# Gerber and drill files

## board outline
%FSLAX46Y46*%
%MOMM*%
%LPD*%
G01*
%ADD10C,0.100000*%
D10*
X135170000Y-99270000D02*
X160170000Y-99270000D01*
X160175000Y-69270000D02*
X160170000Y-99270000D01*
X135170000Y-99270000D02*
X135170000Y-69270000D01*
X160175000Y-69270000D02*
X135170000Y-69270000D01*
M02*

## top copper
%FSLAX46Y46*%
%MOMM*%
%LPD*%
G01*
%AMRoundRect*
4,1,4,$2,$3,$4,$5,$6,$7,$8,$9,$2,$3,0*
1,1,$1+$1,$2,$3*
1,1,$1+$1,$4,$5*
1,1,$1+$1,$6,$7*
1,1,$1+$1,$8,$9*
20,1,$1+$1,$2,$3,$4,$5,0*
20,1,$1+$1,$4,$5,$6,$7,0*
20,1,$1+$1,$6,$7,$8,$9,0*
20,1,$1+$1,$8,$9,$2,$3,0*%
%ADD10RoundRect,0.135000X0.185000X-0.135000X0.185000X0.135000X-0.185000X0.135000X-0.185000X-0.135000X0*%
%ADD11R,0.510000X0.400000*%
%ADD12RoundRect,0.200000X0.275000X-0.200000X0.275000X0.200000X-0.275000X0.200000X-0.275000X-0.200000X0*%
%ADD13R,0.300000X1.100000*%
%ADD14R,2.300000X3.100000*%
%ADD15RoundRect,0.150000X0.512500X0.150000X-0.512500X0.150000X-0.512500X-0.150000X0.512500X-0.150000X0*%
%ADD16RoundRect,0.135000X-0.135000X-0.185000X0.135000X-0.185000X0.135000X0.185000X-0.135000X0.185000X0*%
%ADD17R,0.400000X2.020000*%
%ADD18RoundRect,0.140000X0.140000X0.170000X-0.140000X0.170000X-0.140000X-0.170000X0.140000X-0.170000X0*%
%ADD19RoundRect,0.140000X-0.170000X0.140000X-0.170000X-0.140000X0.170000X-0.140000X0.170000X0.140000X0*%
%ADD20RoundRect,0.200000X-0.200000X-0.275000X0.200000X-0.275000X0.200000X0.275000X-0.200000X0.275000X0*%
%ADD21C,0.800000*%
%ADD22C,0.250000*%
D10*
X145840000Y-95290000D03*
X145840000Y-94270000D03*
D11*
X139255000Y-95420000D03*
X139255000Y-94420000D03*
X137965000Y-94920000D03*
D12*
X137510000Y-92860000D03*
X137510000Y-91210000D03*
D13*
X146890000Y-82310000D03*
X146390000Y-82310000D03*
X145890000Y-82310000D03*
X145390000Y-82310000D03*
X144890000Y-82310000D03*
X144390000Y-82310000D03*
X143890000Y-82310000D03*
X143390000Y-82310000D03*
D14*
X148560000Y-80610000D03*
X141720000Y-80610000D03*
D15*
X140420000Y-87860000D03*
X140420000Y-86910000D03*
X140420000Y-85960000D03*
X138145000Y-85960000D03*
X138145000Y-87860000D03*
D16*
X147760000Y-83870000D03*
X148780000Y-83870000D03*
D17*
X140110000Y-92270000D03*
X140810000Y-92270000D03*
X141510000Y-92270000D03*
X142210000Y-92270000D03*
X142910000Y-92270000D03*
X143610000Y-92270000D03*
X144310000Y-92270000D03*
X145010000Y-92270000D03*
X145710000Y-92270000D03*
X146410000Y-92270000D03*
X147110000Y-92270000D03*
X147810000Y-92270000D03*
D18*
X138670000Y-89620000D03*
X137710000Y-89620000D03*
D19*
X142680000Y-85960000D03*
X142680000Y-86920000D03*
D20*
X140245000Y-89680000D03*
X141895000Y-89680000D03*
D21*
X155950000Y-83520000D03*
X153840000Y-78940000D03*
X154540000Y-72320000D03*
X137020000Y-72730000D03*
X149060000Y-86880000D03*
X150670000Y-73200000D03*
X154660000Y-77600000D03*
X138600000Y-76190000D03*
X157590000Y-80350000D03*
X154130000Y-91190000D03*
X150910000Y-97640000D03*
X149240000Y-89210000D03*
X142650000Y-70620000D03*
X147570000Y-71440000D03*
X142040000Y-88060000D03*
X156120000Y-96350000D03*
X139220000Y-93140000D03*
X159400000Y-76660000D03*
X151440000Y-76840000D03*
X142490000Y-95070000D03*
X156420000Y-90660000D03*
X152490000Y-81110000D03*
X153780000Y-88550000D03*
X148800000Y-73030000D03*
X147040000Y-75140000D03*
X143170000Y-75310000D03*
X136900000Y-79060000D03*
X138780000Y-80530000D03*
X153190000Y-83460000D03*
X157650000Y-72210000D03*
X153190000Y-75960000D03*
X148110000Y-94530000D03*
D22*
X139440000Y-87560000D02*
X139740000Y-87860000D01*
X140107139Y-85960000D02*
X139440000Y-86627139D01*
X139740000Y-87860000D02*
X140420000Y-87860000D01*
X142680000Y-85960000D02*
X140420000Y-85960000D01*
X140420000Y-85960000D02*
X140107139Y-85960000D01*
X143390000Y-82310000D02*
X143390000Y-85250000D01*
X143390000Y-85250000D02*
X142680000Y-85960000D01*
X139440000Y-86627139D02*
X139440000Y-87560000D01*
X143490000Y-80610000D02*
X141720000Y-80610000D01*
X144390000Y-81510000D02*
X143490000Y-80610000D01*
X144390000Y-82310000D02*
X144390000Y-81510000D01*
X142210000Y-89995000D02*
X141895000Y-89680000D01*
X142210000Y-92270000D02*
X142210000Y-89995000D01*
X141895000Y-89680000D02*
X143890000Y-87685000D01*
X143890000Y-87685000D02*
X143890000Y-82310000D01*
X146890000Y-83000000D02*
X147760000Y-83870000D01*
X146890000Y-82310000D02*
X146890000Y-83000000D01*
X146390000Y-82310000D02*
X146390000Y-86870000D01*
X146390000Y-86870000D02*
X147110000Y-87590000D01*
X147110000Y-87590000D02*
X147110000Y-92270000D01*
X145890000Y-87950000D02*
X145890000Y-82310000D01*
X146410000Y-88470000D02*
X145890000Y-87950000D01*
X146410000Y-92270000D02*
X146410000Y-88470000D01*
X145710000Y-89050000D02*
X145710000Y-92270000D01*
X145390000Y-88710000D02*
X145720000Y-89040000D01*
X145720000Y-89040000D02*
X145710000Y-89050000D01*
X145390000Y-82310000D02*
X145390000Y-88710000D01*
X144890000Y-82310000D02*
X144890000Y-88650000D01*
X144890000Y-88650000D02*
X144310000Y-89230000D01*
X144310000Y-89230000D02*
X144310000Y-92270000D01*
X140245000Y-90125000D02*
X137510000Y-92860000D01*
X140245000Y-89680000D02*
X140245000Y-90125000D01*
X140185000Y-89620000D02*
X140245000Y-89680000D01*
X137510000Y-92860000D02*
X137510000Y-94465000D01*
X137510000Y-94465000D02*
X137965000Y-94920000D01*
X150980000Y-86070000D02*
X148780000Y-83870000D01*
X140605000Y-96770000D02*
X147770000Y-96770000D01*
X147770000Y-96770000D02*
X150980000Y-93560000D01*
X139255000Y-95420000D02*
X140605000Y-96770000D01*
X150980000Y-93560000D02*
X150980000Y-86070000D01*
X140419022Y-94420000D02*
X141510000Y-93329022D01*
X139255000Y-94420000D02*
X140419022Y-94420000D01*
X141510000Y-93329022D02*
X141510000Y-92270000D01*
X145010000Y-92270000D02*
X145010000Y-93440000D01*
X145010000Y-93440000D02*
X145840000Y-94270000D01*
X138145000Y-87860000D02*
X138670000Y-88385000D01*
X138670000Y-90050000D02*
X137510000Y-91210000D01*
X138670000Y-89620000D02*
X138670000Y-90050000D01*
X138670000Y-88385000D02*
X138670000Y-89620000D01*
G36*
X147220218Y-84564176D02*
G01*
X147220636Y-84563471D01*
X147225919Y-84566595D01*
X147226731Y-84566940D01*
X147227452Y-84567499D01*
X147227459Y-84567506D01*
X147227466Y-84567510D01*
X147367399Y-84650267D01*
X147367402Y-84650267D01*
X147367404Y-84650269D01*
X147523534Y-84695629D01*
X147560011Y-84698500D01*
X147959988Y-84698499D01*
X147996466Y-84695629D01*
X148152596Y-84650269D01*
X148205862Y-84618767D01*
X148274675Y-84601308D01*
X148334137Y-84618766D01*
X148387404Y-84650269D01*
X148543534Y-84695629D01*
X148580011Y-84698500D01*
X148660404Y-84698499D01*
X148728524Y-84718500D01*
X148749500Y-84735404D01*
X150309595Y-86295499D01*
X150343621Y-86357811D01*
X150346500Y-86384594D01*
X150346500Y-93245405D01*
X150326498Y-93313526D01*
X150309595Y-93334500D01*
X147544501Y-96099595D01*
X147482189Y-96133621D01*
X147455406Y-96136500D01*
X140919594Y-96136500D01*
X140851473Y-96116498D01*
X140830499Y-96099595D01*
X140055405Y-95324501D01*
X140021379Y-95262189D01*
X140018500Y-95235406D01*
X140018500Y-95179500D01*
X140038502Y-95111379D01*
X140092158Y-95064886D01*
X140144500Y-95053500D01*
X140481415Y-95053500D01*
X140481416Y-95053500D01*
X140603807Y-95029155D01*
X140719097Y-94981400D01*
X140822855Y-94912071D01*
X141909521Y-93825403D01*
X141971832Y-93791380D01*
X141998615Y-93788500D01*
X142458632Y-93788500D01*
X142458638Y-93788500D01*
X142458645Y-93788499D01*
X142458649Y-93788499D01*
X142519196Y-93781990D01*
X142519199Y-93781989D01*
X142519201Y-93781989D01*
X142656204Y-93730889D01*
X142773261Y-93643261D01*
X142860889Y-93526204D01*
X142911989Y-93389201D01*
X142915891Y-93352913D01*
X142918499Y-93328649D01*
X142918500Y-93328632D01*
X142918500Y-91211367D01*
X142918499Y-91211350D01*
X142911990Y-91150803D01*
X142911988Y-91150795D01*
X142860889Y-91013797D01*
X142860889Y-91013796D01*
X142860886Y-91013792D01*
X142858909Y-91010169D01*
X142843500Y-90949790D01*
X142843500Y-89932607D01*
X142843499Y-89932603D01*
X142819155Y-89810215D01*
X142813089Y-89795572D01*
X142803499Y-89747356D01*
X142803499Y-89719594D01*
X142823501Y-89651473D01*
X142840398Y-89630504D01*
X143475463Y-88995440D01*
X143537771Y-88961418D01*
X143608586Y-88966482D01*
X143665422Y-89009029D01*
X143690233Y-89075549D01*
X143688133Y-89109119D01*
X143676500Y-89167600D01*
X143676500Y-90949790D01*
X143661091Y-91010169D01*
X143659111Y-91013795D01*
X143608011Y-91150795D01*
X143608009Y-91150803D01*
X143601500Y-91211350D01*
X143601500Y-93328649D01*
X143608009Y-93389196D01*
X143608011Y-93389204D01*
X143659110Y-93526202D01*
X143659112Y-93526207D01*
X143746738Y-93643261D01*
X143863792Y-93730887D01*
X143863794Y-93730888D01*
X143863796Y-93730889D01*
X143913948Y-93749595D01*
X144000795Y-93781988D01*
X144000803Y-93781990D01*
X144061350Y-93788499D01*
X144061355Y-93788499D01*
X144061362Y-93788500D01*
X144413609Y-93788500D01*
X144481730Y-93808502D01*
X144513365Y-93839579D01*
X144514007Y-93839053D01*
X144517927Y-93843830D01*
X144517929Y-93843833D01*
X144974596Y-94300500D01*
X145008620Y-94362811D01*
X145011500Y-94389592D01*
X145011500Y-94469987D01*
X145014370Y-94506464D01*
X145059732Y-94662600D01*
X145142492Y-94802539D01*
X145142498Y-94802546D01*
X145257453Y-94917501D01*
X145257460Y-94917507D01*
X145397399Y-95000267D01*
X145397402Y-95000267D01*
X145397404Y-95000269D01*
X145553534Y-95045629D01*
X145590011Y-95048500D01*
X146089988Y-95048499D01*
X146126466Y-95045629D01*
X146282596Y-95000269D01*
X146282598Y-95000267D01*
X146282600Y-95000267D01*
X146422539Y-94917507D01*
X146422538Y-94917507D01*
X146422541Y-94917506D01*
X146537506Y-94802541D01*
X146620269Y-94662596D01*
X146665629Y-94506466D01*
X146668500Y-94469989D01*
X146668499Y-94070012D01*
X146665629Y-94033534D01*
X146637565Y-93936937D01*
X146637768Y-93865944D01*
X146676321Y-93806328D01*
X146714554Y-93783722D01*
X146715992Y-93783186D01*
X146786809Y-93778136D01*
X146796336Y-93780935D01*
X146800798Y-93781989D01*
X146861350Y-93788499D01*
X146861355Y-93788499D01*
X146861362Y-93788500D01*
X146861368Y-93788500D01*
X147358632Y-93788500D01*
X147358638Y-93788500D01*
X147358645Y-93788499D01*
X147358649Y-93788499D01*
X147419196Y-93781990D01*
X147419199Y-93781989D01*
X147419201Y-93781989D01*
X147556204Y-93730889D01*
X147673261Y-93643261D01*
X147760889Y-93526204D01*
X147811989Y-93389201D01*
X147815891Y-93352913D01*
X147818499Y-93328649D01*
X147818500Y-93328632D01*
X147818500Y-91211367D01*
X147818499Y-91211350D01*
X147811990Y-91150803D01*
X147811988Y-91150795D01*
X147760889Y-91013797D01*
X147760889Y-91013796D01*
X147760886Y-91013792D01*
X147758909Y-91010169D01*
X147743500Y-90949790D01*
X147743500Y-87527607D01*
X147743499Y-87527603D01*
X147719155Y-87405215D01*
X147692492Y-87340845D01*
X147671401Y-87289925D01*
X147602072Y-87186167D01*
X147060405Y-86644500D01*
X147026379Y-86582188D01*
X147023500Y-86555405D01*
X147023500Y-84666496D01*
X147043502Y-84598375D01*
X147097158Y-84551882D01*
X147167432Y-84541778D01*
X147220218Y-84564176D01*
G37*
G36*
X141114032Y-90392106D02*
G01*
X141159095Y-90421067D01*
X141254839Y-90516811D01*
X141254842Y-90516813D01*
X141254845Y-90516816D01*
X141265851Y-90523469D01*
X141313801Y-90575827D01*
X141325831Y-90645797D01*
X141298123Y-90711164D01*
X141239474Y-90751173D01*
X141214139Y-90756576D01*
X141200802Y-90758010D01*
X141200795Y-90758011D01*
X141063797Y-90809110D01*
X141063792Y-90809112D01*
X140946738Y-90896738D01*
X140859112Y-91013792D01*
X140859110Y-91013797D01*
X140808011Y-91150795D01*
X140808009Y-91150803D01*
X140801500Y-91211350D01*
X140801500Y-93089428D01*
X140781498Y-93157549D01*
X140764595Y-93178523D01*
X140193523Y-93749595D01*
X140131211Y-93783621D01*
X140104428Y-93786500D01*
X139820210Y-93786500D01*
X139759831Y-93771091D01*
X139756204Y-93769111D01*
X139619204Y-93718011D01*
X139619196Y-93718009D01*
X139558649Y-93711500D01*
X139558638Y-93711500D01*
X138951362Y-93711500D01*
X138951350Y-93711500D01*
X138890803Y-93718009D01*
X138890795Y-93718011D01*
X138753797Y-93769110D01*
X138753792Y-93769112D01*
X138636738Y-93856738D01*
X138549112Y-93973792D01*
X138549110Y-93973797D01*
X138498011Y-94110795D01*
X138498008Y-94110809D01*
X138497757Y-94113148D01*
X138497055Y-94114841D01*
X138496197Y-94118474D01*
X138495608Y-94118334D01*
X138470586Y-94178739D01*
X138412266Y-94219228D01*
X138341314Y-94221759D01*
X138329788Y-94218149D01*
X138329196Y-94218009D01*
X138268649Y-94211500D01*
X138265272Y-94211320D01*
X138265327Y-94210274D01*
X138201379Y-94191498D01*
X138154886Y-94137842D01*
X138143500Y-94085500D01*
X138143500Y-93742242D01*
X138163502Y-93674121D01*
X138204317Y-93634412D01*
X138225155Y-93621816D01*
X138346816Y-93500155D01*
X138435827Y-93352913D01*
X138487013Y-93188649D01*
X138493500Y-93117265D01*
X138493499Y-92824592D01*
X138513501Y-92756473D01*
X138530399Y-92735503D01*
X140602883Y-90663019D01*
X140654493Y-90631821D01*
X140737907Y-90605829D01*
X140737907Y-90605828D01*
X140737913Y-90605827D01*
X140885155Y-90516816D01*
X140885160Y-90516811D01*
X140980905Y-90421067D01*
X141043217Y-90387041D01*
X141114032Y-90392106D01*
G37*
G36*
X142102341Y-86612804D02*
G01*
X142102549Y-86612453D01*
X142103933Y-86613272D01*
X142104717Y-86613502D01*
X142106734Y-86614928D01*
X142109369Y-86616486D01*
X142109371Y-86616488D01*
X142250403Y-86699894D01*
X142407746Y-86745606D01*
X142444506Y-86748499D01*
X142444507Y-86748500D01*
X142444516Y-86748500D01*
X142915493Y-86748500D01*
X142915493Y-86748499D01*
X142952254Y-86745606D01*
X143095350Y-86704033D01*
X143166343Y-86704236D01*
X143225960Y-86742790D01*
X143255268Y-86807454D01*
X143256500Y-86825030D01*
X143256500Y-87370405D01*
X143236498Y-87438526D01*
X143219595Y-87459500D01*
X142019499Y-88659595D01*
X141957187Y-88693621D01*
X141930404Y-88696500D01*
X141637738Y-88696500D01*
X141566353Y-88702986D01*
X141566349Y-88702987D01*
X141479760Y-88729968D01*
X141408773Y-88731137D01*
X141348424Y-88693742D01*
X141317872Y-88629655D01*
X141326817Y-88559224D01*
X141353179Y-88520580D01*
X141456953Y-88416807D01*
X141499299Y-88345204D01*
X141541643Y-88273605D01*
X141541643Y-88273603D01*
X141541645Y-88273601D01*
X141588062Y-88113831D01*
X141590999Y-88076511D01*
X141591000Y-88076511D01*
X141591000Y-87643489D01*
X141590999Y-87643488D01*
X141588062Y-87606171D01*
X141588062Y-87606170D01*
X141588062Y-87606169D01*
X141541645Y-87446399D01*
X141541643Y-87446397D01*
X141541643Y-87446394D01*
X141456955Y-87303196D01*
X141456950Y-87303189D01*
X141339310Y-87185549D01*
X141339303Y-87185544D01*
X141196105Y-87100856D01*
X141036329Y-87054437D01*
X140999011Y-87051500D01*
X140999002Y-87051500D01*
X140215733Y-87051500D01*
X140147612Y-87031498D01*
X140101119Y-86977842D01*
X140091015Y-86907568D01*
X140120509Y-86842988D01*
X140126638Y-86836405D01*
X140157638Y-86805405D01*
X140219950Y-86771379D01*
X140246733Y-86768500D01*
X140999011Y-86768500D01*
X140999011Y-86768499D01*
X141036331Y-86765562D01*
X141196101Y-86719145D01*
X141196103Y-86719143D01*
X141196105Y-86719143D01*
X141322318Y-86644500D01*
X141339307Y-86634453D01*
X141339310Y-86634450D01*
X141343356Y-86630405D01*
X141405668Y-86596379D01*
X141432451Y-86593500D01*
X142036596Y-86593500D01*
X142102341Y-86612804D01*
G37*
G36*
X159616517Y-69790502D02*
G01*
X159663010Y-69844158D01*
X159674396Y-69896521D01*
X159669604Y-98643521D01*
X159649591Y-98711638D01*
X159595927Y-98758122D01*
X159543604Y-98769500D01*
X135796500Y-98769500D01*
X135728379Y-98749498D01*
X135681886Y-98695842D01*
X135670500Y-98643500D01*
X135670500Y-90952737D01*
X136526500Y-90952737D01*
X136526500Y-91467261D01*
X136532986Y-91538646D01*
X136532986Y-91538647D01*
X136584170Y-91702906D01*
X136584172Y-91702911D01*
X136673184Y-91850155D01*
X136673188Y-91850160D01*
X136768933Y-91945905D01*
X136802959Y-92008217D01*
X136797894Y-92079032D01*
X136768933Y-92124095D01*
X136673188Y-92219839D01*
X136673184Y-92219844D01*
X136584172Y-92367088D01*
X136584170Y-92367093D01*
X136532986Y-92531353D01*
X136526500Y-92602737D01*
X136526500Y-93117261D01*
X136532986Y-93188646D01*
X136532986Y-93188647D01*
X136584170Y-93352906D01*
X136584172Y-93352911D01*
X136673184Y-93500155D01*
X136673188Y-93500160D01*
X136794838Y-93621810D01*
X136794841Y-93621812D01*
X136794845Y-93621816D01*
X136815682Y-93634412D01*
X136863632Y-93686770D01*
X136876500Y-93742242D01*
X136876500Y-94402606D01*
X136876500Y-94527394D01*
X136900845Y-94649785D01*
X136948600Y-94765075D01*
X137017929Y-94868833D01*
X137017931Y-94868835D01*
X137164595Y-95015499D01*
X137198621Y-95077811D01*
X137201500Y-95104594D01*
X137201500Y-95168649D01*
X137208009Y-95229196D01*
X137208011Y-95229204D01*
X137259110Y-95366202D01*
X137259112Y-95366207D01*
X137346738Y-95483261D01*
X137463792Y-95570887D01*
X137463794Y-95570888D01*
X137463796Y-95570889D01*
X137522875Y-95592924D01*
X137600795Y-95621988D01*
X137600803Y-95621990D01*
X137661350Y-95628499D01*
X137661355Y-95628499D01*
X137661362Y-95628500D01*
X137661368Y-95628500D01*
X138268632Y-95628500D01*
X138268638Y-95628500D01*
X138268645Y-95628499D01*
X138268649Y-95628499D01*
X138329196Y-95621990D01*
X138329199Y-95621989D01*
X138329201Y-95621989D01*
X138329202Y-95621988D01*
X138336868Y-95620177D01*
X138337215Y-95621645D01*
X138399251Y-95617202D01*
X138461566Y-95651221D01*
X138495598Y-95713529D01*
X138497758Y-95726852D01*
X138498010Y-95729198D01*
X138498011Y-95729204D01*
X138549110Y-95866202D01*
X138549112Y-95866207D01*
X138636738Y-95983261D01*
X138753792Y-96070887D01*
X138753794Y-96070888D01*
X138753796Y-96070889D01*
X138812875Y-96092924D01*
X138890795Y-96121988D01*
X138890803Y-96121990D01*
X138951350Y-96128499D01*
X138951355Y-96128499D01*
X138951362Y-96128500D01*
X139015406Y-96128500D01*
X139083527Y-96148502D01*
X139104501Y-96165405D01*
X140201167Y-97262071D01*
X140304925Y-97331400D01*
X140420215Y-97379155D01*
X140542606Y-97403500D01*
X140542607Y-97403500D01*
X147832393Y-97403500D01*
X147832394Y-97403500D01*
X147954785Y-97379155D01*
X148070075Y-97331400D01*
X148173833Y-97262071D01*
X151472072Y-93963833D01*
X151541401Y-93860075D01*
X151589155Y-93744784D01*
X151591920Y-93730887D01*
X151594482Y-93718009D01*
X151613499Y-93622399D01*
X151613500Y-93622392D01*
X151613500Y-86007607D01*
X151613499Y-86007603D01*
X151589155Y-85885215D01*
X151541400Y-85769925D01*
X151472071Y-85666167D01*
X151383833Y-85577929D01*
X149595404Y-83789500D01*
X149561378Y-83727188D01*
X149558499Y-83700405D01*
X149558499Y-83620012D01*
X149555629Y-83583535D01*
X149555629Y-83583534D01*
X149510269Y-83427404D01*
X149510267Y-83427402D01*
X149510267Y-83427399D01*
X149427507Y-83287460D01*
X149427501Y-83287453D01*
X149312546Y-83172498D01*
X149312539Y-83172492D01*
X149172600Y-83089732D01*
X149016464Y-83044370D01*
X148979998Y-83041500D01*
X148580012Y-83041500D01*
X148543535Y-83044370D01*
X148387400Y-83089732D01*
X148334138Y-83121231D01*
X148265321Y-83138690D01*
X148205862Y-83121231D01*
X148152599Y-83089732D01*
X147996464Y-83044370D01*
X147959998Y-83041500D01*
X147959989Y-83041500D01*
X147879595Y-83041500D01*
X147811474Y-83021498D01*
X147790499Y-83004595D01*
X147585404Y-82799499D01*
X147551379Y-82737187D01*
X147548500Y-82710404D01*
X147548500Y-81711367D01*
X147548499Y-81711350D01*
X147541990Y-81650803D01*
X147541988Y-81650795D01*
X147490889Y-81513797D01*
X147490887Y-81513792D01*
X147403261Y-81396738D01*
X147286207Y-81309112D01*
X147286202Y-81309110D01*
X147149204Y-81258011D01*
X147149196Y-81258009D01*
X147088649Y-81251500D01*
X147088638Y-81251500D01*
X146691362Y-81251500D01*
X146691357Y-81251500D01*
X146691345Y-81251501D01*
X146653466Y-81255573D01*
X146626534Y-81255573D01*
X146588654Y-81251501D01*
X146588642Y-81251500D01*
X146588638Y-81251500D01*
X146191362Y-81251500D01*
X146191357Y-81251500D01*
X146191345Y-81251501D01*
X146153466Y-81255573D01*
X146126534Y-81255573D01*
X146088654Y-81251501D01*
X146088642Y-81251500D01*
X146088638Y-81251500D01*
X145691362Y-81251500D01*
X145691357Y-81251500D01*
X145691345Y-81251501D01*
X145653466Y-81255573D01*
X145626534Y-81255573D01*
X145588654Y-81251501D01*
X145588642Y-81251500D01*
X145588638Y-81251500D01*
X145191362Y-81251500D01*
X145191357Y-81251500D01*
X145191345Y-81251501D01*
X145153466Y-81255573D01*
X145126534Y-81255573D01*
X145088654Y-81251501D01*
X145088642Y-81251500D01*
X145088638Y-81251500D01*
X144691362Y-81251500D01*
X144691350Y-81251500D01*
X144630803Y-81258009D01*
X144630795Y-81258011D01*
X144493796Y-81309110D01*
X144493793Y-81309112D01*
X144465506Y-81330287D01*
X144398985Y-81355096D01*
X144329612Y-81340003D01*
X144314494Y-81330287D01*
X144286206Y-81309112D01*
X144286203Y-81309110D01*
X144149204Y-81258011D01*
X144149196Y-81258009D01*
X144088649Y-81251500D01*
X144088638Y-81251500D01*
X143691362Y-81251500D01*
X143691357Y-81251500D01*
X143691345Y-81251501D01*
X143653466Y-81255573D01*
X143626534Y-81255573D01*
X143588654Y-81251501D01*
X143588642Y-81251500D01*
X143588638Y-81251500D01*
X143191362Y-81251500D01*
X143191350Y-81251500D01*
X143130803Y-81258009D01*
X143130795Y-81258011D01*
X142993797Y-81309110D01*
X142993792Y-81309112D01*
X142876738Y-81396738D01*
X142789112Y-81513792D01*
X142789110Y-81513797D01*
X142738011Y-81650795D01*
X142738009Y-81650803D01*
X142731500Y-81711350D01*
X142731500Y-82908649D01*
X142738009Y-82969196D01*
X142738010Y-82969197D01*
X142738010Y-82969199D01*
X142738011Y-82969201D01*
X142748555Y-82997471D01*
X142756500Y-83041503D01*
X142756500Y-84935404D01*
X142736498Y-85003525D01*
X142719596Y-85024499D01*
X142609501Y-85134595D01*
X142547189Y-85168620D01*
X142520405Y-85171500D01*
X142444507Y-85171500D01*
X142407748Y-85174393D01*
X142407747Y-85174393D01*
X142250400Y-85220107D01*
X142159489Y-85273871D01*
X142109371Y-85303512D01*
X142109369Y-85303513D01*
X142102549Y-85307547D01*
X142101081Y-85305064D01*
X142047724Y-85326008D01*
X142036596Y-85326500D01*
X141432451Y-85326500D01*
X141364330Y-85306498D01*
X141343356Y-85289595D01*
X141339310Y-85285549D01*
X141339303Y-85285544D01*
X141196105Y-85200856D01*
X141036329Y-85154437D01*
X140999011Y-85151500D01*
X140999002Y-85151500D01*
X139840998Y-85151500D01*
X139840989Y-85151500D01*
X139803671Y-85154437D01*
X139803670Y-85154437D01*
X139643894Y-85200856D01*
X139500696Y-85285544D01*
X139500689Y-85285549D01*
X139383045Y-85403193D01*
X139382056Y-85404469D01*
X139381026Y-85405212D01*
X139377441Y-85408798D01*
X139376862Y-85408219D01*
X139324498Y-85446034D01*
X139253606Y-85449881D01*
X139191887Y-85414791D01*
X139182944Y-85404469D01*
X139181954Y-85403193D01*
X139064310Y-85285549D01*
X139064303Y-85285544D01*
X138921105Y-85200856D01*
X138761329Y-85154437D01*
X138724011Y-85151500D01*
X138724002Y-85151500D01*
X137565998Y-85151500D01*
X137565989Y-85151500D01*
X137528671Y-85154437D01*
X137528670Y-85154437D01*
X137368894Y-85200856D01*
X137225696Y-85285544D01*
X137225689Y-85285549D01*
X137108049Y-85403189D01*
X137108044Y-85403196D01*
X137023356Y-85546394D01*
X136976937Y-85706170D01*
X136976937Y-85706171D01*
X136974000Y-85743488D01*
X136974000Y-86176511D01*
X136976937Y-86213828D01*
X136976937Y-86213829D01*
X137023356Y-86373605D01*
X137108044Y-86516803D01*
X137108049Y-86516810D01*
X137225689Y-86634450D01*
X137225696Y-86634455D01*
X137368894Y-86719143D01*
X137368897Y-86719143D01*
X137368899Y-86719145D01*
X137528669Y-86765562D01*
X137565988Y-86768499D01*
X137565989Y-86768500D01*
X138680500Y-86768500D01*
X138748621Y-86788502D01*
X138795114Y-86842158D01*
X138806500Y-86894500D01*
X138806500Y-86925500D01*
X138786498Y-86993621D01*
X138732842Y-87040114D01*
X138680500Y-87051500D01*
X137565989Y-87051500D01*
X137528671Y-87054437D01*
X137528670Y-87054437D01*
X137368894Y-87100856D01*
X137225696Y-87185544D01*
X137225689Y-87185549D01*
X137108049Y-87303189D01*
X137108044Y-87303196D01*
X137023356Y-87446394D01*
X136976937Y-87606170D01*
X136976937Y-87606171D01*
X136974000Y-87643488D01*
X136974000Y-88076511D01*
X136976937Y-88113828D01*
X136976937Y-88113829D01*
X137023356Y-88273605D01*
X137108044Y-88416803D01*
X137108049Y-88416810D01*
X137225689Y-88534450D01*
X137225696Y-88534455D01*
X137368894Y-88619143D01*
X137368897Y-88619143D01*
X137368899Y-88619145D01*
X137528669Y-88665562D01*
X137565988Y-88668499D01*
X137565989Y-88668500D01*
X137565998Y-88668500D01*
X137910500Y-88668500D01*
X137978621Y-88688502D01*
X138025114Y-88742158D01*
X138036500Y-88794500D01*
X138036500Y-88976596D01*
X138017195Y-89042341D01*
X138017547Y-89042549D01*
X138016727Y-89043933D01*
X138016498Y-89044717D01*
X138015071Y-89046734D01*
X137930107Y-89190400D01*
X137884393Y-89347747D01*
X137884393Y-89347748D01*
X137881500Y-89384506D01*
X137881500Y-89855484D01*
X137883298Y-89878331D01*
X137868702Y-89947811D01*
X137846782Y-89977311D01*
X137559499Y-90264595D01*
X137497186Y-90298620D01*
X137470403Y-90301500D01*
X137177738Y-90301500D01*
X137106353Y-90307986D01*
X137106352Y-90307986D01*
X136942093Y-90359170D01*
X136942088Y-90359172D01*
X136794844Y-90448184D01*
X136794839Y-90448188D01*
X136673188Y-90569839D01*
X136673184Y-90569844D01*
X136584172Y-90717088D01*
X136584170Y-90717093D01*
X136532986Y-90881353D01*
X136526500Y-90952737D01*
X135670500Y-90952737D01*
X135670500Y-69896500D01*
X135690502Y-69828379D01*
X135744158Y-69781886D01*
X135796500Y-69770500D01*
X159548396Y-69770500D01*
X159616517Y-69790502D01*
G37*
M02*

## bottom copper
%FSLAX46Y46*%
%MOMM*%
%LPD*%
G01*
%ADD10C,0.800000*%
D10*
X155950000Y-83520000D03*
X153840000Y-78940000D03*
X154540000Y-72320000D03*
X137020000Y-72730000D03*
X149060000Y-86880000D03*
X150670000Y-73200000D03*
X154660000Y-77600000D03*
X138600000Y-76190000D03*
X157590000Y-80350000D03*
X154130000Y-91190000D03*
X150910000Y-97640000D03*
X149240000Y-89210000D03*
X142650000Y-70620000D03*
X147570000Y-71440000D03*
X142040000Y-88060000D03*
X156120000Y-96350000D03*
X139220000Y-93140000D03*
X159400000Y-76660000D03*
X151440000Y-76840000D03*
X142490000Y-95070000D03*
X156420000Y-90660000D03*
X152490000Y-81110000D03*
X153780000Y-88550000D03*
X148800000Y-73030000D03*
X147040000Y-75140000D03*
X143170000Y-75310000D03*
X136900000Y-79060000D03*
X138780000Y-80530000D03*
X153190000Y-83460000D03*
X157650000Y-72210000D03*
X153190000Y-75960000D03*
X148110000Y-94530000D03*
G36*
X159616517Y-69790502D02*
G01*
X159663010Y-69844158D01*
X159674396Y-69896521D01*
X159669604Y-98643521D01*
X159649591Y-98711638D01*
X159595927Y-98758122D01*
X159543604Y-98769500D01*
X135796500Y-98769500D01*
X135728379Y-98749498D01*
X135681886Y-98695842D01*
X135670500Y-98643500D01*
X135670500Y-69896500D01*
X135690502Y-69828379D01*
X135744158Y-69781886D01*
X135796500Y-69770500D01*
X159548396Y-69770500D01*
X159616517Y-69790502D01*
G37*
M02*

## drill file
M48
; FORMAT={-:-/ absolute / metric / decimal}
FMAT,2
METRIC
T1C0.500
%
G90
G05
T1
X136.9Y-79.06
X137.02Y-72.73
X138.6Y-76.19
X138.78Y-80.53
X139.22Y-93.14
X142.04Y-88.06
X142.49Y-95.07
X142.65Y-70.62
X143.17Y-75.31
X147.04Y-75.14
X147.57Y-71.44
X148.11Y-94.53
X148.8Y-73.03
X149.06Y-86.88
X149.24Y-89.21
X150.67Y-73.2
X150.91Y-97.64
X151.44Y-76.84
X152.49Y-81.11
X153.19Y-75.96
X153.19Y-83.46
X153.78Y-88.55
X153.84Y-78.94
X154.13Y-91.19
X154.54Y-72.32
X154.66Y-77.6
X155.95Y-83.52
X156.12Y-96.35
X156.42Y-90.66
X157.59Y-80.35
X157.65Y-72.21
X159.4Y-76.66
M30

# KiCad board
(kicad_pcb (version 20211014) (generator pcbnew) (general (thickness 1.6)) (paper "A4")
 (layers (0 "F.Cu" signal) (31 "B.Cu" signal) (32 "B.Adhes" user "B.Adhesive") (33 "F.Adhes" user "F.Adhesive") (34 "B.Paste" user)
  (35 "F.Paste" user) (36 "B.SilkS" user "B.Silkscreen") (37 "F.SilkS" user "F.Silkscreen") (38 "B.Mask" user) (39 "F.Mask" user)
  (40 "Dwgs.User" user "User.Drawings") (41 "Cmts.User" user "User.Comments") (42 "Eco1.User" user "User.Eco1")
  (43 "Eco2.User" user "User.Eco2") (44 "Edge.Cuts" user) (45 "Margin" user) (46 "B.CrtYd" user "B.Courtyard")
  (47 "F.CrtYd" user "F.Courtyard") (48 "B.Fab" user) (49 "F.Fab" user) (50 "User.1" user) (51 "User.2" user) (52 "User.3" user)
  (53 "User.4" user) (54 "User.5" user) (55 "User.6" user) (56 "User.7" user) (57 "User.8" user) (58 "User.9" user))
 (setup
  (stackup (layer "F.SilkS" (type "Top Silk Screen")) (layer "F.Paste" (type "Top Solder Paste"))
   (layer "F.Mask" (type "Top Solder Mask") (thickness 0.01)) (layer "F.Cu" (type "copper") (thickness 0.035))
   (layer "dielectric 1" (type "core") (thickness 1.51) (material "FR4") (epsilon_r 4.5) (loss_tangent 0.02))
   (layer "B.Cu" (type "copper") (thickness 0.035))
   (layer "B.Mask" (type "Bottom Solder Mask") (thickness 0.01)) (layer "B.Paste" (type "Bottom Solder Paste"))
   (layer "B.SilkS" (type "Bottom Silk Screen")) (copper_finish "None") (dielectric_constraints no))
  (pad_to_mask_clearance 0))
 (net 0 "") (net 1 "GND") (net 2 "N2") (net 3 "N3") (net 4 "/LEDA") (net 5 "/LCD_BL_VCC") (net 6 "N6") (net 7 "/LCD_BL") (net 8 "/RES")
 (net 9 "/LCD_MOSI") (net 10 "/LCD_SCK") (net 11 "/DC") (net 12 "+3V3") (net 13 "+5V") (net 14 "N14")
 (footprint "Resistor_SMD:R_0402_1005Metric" (layer "F.Cu") (at 145.84 94.78 90)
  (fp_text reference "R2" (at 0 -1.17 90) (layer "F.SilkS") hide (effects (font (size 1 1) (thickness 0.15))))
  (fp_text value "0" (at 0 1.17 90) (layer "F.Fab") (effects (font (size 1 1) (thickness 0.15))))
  (pad "1" smd roundrect (at -0.51 0 90) (size 0.54 0.64) (layers "F.Cu" "F.Paste" "F.Mask") (roundrect_rratio 0.25) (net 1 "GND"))
  (pad "2" smd roundrect (at 0.51 0 90) (size 0.54 0.64) (layers "F.Cu" "F.Paste" "F.Mask") (roundrect_rratio 0.25) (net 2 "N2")))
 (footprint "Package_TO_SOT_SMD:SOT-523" (layer "F.Cu") (at 138.61 94.92 180)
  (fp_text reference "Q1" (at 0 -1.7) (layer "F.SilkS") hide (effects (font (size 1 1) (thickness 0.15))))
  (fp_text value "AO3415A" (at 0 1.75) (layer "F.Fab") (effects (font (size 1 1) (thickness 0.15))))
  (pad "1" smd rect (at -0.645 -0.5) (size 0.51 0.4) (layers "F.Cu" "F.Paste" "F.Mask") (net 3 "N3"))
  (pad "2" smd rect (at -0.645 0.5) (size 0.51 0.4) (layers "F.Cu" "F.Paste" "F.Mask") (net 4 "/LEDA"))
  (pad "3" smd rect (at 0.645 0) (size 0.51 0.4) (layers "F.Cu" "F.Paste" "F.Mask") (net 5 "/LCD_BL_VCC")))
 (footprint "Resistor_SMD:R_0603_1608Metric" (layer "F.Cu") (at 137.51 92.035 90)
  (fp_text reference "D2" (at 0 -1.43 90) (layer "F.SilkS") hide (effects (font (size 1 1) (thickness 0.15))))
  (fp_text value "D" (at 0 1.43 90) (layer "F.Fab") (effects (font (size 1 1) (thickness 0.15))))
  (pad "1" smd roundrect (at -0.825 0 90) (size 0.8 0.95) (layers "F.Cu" "F.Paste" "F.Mask") (roundrect_rratio 0.25) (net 5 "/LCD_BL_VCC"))
  (pad "2" smd roundrect (at 0.825 0 90) (size 0.8 0.95) (layers "F.Cu" "F.Paste" "F.Mask") (roundrect_rratio 0.25) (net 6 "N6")))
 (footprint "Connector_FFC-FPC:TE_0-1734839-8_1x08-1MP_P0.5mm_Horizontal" (layer "F.Cu") (at 145.14 80.96 180)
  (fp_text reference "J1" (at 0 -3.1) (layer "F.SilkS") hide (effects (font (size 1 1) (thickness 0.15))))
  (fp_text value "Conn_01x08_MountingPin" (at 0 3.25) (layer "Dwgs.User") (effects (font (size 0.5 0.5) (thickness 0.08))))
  (pad "1" smd rect (at -1.75 -1.35 180) (size 0.3 1.1) (layers "F.Cu" "F.Paste" "F.Mask") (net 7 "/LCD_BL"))
  (pad "2" smd rect (at -1.25 -1.35 180) (size 0.3 1.1) (layers "F.Cu" "F.Paste" "F.Mask") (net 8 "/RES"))
  (pad "3" smd rect (at -0.75 -1.35 180) (size 0.3 1.1) (layers "F.Cu" "F.Paste" "F.Mask") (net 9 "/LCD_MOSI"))
  (pad "4" smd rect (at -0.25 -1.35 180) (size 0.3 1.1) (layers "F.Cu" "F.Paste" "F.Mask") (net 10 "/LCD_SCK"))
  (pad "5" smd rect (at 0.25 -1.35 180) (size 0.3 1.1) (layers "F.Cu" "F.Paste" "F.Mask") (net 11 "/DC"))
  (pad "6" smd rect (at 0.75 -1.35 180) (size 0.3 1.1) (layers "F.Cu" "F.Paste" "F.Mask") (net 1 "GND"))
  (pad "7" smd rect (at 1.25 -1.35 180) (size 0.3 1.1) (layers "F.Cu" "F.Paste" "F.Mask") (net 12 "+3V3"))
  (pad "8" smd rect (at 1.75 -1.35 180) (size 0.3 1.1) (layers "F.Cu" "F.Paste" "F.Mask") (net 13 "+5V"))
  (pad "MP" smd rect (at -3.42 0.35 180) (size 2.3 3.1) (layers "F.Cu" "F.Paste" "F.Mask") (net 1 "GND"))
  (pad "MP" smd rect (at 3.42 0.35 180) (size 2.3 3.1) (layers "F.Cu" "F.Paste" "F.Mask") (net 1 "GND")))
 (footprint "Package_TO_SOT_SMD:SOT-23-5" (layer "F.Cu") (at 139.2825 86.91 180)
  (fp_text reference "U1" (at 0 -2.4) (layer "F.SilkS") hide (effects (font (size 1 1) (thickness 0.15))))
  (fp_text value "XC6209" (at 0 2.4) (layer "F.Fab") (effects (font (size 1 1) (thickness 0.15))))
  (pad "1" smd roundrect (at -1.1375 -0.95 180) (size 1.325 0.6) (layers "F.Cu" "F.Paste" "F.Mask") (roundrect_rratio 0.25) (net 13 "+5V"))
  (pad "2" smd roundrect (at -1.1375 0 180) (size 1.325 0.6) (layers "F.Cu" "F.Paste" "F.Mask") (roundrect_rratio 0.25) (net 1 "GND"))
  (pad "3" smd roundrect (at -1.1375 0.95 180) (size 1.325 0.6) (layers "F.Cu" "F.Paste" "F.Mask") (roundrect_rratio 0.25) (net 13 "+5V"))
  (pad "4" smd roundrect (at 1.1375 0.95 180) (size 1.325 0.6) (layers "F.Cu" "F.Paste" "F.Mask") (roundrect_rratio 0.25) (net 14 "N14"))
  (pad "5" smd roundrect (at 1.1375 -0.95 180) (size 1.325 0.6) (layers "F.Cu" "F.Paste" "F.Mask") (roundrect_rratio 0.25) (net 6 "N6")))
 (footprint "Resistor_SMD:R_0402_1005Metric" (layer "F.Cu") (at 148.27 83.87)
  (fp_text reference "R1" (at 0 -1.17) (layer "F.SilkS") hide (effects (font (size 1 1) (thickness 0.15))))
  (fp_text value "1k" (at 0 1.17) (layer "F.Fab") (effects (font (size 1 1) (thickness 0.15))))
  (pad "1" smd roundrect (at -0.51 0) (size 0.54 0.64) (layers "F.Cu" "F.Paste" "F.Mask") (roundrect_rratio 0.25) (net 7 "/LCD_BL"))
  (pad "2" smd roundrect (at 0.51 0) (size 0.54 0.64) (layers "F.Cu" "F.Paste" "F.Mask") (roundrect_rratio 0.25) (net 3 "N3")))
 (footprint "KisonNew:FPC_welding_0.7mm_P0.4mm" (layer "F.Cu") (at 143.98 91.13)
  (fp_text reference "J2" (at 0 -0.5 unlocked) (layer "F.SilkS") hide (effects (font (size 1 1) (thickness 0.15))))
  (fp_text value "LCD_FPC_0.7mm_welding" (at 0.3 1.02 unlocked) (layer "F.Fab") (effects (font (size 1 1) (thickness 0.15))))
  (pad "1" smd rect (at -3.87 1.14) (size 0.4 2.02) (layers "F.Cu" "F.Paste" "F.Mask") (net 1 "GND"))
  (pad "2" smd rect (at -3.17 1.14) (size 0.4 2.02) (layers "F.Cu" "F.Paste" "F.Mask") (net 1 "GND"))
  (pad "3" smd rect (at -2.47 1.14) (size 0.4 2.02) (layers "F.Cu" "F.Paste" "F.Mask") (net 4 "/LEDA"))
  (pad "4" smd rect (at -1.77 1.14) (size 0.4 2.02) (layers "F.Cu" "F.Paste" "F.Mask") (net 12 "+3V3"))
  (pad "5" smd rect (at -1.07 1.14) (size 0.4 2.02) (layers "F.Cu" "F.Paste" "F.Mask") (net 1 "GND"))
  (pad "6" smd rect (at -0.37 1.14) (size 0.4 2.02) (layers "F.Cu" "F.Paste" "F.Mask") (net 1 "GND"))
  (pad "7" smd rect (at 0.33 1.14) (size 0.4 2.02) (layers "F.Cu" "F.Paste" "F.Mask") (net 11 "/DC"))
  (pad "8" smd rect (at 1.03 1.14) (size 0.4 2.02) (layers "F.Cu" "F.Paste" "F.Mask") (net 2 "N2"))
  (pad "9" smd rect (at 1.73 1.14) (size 0.4 2.02) (layers "F.Cu" "F.Paste" "F.Mask") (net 10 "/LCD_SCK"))
  (pad "10" smd rect (at 2.43 1.14) (size 0.4 2.02) (layers "F.Cu" "F.Paste" "F.Mask") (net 9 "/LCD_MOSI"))
  (pad "11" smd rect (at 3.13 1.14) (size 0.4 2.02) (layers "F.Cu" "F.Paste" "F.Mask") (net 8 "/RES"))
  (pad "12" smd rect (at 3.83 1.14) (size 0.4 2.02) (layers "F.Cu" "F.Paste" "F.Mask") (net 1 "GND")))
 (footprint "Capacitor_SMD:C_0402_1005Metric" (layer "F.Cu") (at 138.19 89.62 180)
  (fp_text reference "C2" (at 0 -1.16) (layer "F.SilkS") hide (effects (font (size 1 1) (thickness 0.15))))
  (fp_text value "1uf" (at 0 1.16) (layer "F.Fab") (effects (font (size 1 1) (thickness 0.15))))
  (pad "1" smd roundrect (at -0.48 0 180) (size 0.56 0.62) (layers "F.Cu" "F.Paste" "F.Mask") (roundrect_rratio 0.25) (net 6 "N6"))
  (pad "2" smd roundrect (at 0.48 0 180) (size 0.56 0.62) (layers "F.Cu" "F.Paste" "F.Mask") (roundrect_rratio 0.25) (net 1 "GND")))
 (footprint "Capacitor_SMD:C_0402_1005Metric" (layer "F.Cu") (at 142.68 86.44 -90)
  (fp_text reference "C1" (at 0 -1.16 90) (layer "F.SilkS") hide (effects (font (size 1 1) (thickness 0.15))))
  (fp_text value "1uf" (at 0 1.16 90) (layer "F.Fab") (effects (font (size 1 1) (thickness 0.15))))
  (pad "1" smd roundrect (at -0.48 0 270) (size 0.56 0.62) (layers "F.Cu" "F.Paste" "F.Mask") (roundrect_rratio 0.25) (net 13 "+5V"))
  (pad "2" smd roundrect (at 0.48 0 270) (size 0.56 0.62) (layers "F.Cu" "F.Paste" "F.Mask") (roundrect_rratio 0.25) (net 1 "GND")))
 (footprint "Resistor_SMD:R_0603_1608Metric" (layer "F.Cu") (at 141.07 89.68)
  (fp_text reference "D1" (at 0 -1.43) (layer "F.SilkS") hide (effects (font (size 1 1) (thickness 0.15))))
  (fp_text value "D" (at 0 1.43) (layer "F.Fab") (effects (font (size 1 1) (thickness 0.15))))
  (pad "1" smd roundrect (at -0.825 0) (size 0.8 0.95) (layers "F.Cu" "F.Paste" "F.Mask") (roundrect_rratio 0.25) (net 5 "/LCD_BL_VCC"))
  (pad "2" smd roundrect (at 0.825 0) (size 0.8 0.95) (layers "F.Cu" "F.Paste" "F.Mask") (roundrect_rratio 0.25) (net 12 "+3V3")))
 (gr_line (start 135.17 99.27) (end 160.17 99.27) (layer "Edge.Cuts") (width 0.1))
 (gr_line (start 160.175 69.27) (end 160.17 99.27) (layer "Edge.Cuts") (width 0.1))
 (gr_line (start 135.17 99.27) (end 135.17 69.27) (layer "Edge.Cuts") (width 0.1))
 (gr_line (start 160.175 69.27) (end 135.17 69.27) (layer "Edge.Cuts") (width 0.1))
 (segment (start 139.44 87.56) (end 139.74 87.86) (width 0.25) (layer "F.Cu") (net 13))
 (segment (start 140.107139 85.96) (end 139.44 86.627139) (width 0.25) (layer "F.Cu") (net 13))
 (segment (start 139.74 87.86) (end 140.42 87.86) (width 0.25) (layer "F.Cu") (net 13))
 (segment (start 142.68 85.96) (end 140.42 85.96) (width 0.25) (layer "F.Cu") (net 13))
 (segment (start 140.42 85.96) (end 140.107139 85.96) (width 0.25) (layer "F.Cu") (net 13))
 (segment (start 143.39 82.31) (end 143.39 85.25) (width 0.25) (layer "F.Cu") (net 13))
 (segment (start 143.39 85.25) (end 142.68 85.96) (width 0.25) (layer "F.Cu") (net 13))
 (segment (start 139.44 86.627139) (end 139.44 87.56) (width 0.25) (layer "F.Cu") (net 13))
 (segment (start 143.49 80.61) (end 141.72 80.61) (width 0.25) (layer "F.Cu") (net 1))
 (segment (start 144.39 81.51) (end 143.49 80.61) (width 0.25) (layer "F.Cu") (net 1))
 (segment (start 144.39 82.31) (end 144.39 81.51) (width 0.25) (layer "F.Cu") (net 1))
 (via (at 155.95 83.52) (size 0.8) (drill 0.5) (layers "F.Cu" "B.Cu") (free) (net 1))
 (via (at 153.84 78.94) (size 0.8) (drill 0.5) (layers "F.Cu" "B.Cu") (free) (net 1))
 (via (at 154.54 72.32) (size 0.8) (drill 0.5) (layers "F.Cu" "B.Cu") (free) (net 1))
 (via (at 137.02 72.73) (size 0.8) (drill 0.5) (layers "F.Cu" "B.Cu") (free) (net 1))
 (via (at 149.06 86.88) (size 0.8) (drill 0.5) (layers "F.Cu" "B.Cu") (free) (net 1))
 (via (at 150.67 73.2) (size 0.8) (drill 0.5) (layers "F.Cu" "B.Cu") (free) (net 1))
 (via (at 154.66 77.6) (size 0.8) (drill 0.5) (layers "F.Cu" "B.Cu") (free) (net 1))
 (via (at 138.6 76.19) (size 0.8) (drill 0.5) (layers "F.Cu" "B.Cu") (free) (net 1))
 (via (at 157.59 80.35) (size 0.8) (drill 0.5) (layers "F.Cu" "B.Cu") (free) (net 1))
 (via (at 154.13 91.19) (size 0.8) (drill 0.5) (layers "F.Cu" "B.Cu") (free) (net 1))
 (via (at 150.91 97.64) (size 0.8) (drill 0.5) (layers "F.Cu" "B.Cu") (free) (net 1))
 (via (at 149.24 89.21) (size 0.8) (drill 0.5) (layers "F.Cu" "B.Cu") (free) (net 1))
 (via (at 142.65 70.62) (size 0.8) (drill 0.5) (layers "F.Cu" "B.Cu") (free) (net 1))
 (via (at 147.57 71.44) (size 0.8) (drill 0.5) (layers "F.Cu" "B.Cu") (free) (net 1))
 (via (at 142.04 88.06) (size 0.8) (drill 0.5) (layers "F.Cu" "B.Cu") (free) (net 1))
 (via (at 156.12 96.35) (size 0.8) (drill 0.5) (layers "F.Cu" "B.Cu") (free) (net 1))
 (via (at 139.22 93.14) (size 0.8) (drill 0.5) (layers "F.Cu" "B.Cu") (free) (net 1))
 (via (at 159.4 76.66) (size 0.8) (drill 0.5) (layers "F.Cu" "B.Cu") (free) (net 1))
 (via (at 151.44 76.84) (size 0.8) (drill 0.5) (layers "F.Cu" "B.Cu") (free) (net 1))
 (via (at 142.49 95.07) (size 0.8) (drill 0.5) (layers "F.Cu" "B.Cu") (free) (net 1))
 (via (at 156.42 90.66) (size 0.8) (drill 0.5) (layers "F.Cu" "B.Cu") (free) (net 1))
 (via (at 152.49 81.11) (size 0.8) (drill 0.5) (layers "F.Cu" "B.Cu") (free) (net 1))
 (via (at 153.78 88.55) (size 0.8) (drill 0.5) (layers "F.Cu" "B.Cu") (free) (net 1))
 (via (at 148.8 73.03) (size 0.8) (drill 0.5) (layers "F.Cu" "B.Cu") (free) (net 1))
 (via (at 147.04 75.14) (size 0.8) (drill 0.5) (layers "F.Cu" "B.Cu") (free) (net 1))
 (via (at 143.17 75.31) (size 0.8) (drill 0.5) (layers "F.Cu" "B.Cu") (free) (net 1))
 (via (at 136.9 79.06) (size 0.8) (drill 0.5) (layers "F.Cu" "B.Cu") (free) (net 1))
 (via (at 138.78 80.53) (size 0.8) (drill 0.5) (layers "F.Cu" "B.Cu") (free) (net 1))
 (via (at 153.19 83.46) (size 0.8) (drill 0.5) (layers "F.Cu" "B.Cu") (free) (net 1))
 (via (at 157.65 72.21) (size 0.8) (drill 0.5) (layers "F.Cu" "B.Cu") (free) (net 1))
 (via (at 153.19 75.96) (size 0.8) (drill 0.5) (layers "F.Cu" "B.Cu") (free) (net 1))
 (via (at 148.11 94.53) (size 0.8) (drill 0.5) (layers "F.Cu" "B.Cu") (free) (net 1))
 (segment (start 142.21 89.995) (end 141.895 89.68) (width 0.25) (layer "F.Cu") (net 12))
 (segment (start 142.21 92.27) (end 142.21 89.995) (width 0.25) (layer "F.Cu") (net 12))
 (segment (start 141.895 89.68) (end 143.89 87.685) (width 0.25) (layer "F.Cu") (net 12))
 (segment (start 143.89 87.685) (end 143.89 82.31) (width 0.25) (layer "F.Cu") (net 12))
 (segment (start 146.89 83) (end 147.76 83.87) (width 0.25) (layer "F.Cu") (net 7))
 (segment (start 146.89 82.31) (end 146.89 83) (width 0.25) (layer "F.Cu") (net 7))
 (segment (start 146.39 82.31) (end 146.39 86.87) (width 0.25) (layer "F.Cu") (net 8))
 (segment (start 146.39 86.87) (end 147.11 87.59) (width 0.25) (layer "F.Cu") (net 8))
 (segment (start 147.11 87.59) (end 147.11 92.27) (width 0.25) (layer "F.Cu") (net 8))
 (segment (start 145.89 87.95) (end 145.89 82.31) (width 0.25) (layer "F.Cu") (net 9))
 (segment (start 146.41 88.47) (end 145.89 87.95) (width 0.25) (layer "F.Cu") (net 9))
 (segment (start 146.41 92.27) (end 146.41 88.47) (width 0.25) (layer "F.Cu") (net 9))
 (segment (start 145.71 89.05) (end 145.71 92.27) (width 0.25) (layer "F.Cu") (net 10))
 (segment (start 145.39 88.71) (end 145.72 89.04) (width 0.25) (layer "F.Cu") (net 10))
 (segment (start 145.72 89.04) (end 145.71 89.05) (width 0.25) (layer "F.Cu") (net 10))
 (segment (start 145.39 82.31) (end 145.39 88.71) (width 0.25) (layer "F.Cu") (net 10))
 (segment (start 144.89 82.31) (end 144.89 88.65) (width 0.25) (layer "F.Cu") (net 11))
 (segment (start 144.89 88.65) (end 144.31 89.23) (width 0.25) (layer "F.Cu") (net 11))
 (segment (start 144.31 89.23) (end 144.31 92.27) (width 0.25) (layer "F.Cu") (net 11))
 (segment (start 140.245 90.125) (end 137.51 92.86) (width 0.25) (layer "F.Cu") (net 5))
 (segment (start 140.245 89.68) (end 140.245 90.125) (width 0.25) (layer "F.Cu") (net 5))
 (segment (start 140.185 89.62) (end 140.245 89.68) (width 0.25) (layer "F.Cu") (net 5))
 (segment (start 137.51 92.86) (end 137.51 94.465) (width 0.25) (layer "F.Cu") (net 5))
 (segment (start 137.51 94.465) (end 137.965 94.92) (width 0.25) (layer "F.Cu") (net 5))
 (segment (start 150.98 86.07) (end 148.78 83.87) (width 0.25) (layer "F.Cu") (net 3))
 (segment (start 140.605 96.77) (end 147.77 96.77) (width 0.25) (layer "F.Cu") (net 3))
 (segment (start 147.77 96.77) (end 150.98 93.56) (width 0.25) (layer "F.Cu") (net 3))
 (segment (start 139.255 95.42) (end 140.605 96.77) (width 0.25) (layer "F.Cu") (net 3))
 (segment (start 150.98 93.56) (end 150.98 86.07) (width 0.25) (layer "F.Cu") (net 3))
 (segment (start 140.419022 94.42) (end 141.51 93.329022) (width 0.25) (layer "F.Cu") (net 4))
 (segment (start 139.255 94.42) (end 140.419022 94.42) (width 0.25) (layer "F.Cu") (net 4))
 (segment (start 141.51 93.329022) (end 141.51 92.27) (width 0.25) (layer "F.Cu") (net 4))
 (segment (start 145.01 92.27) (end 145.01 93.44) (width 0.25) (layer "F.Cu") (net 2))
 (segment (start 145.01 93.44) (end 145.84 94.27) (width 0.25) (layer "F.Cu") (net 2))
 (segment (start 138.145 87.86) (end 138.67 88.385) (width 0.25) (layer "F.Cu") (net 6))
 (segment (start 138.67 90.05) (end 137.51 91.21) (width 0.25) (layer "F.Cu") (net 6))
 (segment (start 138.67 89.62) (end 138.67 90.05) (width 0.25) (layer "F.Cu") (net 6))
 (segment (start 138.67 88.385) (end 138.67 89.62) (width 0.25) (layer "F.Cu") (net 6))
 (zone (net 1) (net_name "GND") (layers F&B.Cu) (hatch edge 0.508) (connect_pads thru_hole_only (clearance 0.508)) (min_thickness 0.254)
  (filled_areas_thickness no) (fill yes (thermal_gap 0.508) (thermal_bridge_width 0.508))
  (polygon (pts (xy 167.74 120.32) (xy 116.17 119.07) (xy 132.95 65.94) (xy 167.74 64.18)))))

